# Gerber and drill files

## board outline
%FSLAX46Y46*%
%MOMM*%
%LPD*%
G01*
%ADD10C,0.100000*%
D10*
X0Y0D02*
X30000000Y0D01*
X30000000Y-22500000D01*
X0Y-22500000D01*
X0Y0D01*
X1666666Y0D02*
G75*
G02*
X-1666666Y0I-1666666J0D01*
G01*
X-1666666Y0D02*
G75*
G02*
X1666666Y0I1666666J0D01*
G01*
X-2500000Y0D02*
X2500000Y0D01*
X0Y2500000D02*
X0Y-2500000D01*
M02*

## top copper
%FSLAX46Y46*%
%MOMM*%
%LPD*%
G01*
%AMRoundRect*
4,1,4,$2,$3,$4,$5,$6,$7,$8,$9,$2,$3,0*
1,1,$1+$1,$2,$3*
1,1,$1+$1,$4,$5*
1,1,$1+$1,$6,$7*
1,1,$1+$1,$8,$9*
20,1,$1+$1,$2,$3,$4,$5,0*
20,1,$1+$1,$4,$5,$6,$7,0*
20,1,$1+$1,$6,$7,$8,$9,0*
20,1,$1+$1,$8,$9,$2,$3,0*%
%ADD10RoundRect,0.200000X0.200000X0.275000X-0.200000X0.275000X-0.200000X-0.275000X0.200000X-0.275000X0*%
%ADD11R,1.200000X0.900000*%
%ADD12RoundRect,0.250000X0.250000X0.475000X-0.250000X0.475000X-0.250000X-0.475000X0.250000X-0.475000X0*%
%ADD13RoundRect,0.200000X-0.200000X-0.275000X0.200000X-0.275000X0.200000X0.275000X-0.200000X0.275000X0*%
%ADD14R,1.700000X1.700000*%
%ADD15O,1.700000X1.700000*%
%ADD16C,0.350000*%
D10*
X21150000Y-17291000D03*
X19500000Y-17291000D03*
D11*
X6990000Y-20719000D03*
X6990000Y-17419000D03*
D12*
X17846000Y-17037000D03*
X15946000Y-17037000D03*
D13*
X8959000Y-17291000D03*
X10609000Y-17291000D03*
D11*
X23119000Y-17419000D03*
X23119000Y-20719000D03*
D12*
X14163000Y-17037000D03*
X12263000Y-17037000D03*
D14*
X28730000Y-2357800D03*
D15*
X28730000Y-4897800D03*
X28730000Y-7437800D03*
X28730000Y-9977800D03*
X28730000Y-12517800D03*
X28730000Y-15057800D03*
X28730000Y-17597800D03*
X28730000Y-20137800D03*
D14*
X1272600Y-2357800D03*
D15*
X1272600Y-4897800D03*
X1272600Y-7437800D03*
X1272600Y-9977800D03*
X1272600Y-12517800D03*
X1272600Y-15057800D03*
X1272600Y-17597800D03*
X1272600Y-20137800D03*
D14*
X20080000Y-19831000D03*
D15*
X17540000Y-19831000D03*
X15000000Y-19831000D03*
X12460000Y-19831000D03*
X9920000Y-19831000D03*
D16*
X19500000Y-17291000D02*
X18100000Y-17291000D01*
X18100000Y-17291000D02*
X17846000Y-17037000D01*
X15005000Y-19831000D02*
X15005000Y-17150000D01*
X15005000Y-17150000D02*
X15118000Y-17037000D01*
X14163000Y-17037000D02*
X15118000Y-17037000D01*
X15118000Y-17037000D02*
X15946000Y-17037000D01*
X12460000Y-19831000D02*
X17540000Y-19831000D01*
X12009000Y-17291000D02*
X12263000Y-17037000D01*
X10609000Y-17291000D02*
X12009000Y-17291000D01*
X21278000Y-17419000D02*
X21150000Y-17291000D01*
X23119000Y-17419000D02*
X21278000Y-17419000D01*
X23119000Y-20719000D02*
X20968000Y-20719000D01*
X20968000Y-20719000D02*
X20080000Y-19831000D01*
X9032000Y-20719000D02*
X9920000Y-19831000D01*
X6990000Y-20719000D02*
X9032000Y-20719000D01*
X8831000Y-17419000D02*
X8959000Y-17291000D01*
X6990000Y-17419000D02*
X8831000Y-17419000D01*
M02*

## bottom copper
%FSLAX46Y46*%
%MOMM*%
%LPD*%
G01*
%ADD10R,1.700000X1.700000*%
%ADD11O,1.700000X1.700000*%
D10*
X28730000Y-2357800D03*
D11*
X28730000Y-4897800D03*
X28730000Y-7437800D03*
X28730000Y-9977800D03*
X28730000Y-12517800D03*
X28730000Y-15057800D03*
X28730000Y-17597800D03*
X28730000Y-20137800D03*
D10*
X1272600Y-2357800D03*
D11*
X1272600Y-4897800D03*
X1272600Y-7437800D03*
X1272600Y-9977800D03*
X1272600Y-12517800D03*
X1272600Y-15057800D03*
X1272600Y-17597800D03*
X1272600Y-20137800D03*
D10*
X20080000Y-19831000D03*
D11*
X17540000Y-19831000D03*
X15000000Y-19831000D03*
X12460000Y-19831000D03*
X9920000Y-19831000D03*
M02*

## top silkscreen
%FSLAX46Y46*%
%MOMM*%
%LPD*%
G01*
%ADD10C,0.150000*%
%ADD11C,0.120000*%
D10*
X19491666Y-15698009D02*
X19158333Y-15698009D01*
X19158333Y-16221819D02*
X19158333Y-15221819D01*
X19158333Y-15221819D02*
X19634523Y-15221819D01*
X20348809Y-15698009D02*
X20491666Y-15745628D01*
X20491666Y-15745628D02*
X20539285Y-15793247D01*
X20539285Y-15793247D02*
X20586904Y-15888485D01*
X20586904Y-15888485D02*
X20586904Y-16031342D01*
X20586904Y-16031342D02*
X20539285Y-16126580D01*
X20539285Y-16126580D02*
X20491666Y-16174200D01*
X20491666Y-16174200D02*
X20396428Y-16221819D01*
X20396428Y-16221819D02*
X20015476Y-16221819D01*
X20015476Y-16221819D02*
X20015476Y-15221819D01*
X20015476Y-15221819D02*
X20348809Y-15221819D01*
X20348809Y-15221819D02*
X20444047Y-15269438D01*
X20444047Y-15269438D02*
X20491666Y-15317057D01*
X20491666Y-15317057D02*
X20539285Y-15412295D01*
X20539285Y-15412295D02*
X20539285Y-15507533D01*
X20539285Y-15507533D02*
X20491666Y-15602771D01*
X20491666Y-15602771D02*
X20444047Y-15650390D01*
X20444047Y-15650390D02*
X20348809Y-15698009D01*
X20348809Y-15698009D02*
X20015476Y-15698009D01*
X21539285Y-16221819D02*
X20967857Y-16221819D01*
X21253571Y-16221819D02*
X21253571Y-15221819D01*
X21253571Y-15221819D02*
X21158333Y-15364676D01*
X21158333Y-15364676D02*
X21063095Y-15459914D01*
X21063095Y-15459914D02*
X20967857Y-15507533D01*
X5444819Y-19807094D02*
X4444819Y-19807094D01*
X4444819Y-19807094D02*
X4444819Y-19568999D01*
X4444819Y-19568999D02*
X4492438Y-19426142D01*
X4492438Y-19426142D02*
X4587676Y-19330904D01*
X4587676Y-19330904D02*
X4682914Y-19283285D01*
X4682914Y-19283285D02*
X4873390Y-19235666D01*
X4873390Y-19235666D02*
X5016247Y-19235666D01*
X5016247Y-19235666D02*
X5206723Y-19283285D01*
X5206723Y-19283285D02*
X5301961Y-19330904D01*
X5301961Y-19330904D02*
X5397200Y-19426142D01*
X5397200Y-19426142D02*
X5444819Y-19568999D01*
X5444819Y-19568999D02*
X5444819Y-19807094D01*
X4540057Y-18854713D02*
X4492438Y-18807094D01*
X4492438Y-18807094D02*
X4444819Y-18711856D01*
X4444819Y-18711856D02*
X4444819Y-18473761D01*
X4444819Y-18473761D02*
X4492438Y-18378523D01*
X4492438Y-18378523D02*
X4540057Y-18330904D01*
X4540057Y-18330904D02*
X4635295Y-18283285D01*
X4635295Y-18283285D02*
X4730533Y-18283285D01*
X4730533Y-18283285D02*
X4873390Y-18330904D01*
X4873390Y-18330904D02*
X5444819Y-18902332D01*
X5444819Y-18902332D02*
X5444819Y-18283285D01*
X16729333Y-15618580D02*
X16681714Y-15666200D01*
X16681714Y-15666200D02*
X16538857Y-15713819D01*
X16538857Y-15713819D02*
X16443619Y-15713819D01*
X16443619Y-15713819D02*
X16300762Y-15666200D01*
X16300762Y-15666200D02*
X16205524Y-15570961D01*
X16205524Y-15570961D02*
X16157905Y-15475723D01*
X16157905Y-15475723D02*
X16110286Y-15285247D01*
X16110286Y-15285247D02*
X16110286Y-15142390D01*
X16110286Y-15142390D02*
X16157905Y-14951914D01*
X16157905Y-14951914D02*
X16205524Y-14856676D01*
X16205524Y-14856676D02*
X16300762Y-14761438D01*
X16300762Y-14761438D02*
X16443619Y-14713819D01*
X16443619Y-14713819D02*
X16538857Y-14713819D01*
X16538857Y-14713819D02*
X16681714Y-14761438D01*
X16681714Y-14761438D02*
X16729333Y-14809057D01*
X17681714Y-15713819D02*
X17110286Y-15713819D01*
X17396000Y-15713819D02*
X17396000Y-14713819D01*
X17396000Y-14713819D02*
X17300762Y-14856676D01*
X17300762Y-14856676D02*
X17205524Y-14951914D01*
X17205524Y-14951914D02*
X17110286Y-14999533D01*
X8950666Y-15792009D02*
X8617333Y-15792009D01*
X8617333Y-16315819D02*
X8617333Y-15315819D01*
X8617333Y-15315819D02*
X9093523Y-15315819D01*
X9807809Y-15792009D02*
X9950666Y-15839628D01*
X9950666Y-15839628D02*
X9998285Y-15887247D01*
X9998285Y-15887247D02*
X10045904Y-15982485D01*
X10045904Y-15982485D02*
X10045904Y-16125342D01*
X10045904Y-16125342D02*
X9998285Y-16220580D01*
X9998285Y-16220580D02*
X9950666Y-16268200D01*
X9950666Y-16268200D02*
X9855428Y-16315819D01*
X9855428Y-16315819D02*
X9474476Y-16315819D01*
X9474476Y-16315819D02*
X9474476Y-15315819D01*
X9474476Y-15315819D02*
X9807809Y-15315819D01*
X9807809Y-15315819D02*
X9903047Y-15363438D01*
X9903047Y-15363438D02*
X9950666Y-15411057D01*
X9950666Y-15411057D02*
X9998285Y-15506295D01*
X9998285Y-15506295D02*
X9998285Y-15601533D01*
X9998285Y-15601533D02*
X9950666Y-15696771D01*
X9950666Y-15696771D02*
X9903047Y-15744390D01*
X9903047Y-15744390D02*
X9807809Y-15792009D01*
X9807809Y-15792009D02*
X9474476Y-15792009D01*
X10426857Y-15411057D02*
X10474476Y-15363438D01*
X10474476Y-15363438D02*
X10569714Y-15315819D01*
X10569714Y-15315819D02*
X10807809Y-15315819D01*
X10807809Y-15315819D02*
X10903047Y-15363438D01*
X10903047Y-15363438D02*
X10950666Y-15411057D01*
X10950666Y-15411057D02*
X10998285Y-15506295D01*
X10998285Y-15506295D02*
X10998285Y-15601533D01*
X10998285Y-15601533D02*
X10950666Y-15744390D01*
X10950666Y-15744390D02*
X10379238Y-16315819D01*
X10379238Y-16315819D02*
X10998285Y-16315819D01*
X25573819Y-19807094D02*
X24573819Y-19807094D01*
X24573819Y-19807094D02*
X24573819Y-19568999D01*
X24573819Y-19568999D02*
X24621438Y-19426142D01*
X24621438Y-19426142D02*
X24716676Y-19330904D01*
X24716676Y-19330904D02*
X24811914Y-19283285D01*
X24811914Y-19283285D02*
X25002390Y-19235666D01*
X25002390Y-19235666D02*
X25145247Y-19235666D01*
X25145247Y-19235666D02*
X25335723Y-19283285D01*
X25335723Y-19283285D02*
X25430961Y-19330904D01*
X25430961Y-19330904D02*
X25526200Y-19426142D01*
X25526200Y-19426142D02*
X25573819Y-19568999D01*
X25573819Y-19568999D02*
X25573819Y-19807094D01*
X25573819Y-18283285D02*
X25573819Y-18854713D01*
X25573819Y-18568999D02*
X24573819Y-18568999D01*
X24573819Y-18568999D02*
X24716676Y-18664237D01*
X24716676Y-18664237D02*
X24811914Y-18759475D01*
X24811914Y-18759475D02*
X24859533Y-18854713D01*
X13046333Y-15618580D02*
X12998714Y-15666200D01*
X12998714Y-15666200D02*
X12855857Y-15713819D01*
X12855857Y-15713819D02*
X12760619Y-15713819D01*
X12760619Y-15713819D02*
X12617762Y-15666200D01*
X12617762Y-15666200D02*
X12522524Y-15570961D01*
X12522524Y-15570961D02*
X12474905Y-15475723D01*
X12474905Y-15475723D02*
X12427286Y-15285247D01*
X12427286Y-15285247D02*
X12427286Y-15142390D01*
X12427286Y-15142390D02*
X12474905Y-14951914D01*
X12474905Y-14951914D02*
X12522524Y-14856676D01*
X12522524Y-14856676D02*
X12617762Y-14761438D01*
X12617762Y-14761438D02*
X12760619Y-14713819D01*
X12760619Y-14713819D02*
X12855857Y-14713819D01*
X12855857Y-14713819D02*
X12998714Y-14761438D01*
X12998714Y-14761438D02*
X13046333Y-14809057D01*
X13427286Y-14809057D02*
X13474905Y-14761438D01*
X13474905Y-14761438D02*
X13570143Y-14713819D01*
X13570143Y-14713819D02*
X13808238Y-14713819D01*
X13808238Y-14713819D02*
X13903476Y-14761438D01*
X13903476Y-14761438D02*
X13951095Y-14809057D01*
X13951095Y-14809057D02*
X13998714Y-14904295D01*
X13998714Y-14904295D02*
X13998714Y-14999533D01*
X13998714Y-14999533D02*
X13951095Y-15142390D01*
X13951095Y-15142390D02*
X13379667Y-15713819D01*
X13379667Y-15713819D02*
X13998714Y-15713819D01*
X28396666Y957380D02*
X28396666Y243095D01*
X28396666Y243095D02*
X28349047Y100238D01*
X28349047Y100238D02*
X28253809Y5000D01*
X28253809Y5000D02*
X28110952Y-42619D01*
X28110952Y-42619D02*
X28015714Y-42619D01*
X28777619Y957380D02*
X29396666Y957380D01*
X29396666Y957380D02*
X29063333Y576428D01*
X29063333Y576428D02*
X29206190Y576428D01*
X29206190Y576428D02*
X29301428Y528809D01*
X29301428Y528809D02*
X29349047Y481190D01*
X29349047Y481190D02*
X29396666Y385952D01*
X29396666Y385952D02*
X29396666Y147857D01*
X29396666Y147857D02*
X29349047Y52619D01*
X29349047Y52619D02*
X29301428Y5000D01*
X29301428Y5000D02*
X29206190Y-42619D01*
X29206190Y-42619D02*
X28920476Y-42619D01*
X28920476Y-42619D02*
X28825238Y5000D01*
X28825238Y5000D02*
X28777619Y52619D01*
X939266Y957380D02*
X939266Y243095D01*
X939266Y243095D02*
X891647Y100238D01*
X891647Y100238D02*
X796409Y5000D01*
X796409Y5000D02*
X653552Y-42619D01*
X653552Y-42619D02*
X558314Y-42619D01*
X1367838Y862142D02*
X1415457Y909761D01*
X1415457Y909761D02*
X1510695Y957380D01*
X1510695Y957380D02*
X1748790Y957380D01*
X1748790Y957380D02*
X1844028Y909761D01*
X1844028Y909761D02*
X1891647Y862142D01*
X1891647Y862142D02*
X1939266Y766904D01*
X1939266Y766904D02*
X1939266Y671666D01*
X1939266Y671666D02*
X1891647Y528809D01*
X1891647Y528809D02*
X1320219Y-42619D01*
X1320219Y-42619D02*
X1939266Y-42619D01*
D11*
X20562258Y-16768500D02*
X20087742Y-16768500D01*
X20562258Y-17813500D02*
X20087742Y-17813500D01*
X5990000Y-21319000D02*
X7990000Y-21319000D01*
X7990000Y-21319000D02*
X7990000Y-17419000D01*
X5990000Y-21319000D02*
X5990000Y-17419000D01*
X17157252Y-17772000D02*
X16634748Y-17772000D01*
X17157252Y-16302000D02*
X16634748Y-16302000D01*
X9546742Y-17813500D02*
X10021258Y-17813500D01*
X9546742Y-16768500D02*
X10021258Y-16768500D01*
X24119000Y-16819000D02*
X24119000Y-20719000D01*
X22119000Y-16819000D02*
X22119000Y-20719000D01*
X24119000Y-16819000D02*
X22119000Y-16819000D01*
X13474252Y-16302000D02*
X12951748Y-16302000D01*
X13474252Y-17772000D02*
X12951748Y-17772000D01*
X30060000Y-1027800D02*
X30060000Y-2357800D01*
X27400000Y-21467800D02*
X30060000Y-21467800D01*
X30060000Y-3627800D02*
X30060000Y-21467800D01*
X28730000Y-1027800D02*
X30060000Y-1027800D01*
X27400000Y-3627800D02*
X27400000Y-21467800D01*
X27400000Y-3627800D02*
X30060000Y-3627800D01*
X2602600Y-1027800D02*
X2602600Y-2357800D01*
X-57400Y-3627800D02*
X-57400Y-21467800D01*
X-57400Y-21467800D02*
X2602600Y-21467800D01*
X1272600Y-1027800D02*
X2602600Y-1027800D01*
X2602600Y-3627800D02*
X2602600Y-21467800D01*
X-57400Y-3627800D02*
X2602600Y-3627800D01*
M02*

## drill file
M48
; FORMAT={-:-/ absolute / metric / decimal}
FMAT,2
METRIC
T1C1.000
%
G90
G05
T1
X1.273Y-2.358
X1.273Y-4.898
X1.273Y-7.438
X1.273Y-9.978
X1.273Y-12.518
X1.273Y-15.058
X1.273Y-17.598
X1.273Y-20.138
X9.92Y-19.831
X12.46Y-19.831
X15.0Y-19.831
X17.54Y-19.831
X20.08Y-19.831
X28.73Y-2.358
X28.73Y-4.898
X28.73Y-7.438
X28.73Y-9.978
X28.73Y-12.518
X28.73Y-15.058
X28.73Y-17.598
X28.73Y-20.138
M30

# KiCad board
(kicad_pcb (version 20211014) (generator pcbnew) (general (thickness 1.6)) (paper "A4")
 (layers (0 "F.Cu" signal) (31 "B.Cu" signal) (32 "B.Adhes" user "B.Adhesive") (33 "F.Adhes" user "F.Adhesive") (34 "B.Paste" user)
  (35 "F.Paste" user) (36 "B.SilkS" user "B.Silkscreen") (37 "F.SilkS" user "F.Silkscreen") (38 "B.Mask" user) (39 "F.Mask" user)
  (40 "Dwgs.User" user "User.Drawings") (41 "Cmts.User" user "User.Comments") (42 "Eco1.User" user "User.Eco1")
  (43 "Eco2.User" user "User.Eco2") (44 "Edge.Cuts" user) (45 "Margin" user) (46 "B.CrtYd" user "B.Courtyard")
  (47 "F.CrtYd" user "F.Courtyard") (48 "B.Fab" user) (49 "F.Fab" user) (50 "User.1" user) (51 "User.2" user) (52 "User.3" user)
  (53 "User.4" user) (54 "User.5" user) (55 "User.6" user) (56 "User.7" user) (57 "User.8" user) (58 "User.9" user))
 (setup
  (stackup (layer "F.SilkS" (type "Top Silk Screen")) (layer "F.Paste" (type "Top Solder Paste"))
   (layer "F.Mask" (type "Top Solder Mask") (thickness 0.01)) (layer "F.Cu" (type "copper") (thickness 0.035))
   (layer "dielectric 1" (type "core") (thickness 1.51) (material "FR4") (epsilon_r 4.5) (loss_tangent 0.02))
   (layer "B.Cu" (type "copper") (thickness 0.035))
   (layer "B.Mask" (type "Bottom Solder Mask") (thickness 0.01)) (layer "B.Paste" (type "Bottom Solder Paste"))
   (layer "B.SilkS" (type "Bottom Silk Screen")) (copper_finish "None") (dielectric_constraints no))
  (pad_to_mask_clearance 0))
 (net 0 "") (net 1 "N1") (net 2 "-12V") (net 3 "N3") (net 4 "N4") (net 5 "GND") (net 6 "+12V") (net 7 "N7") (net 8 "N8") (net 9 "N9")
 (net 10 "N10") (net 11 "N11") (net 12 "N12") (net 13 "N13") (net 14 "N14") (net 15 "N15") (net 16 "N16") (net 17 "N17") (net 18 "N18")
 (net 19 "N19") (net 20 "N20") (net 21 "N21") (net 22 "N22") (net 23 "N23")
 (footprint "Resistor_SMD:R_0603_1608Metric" (layer "F.Cu") (at 20.325 17.291 180)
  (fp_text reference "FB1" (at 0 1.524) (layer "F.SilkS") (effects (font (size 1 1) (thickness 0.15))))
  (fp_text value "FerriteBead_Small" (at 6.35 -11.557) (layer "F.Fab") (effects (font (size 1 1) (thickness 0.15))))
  (fp_line (start -0.237258 0.5225) (end 0.237258 0.5225) (layer "F.SilkS") (width 0.12))
  (fp_line (start -0.237258 -0.5225) (end 0.237258 -0.5225) (layer "F.SilkS") (width 0.12))
  (pad "1" smd roundrect (at -0.825 0 180) (size 0.8 0.95) (layers "F.Cu" "F.Paste" "F.Mask") (roundrect_rratio 0.25) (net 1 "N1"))
  (pad "2" smd roundrect (at 0.825 0 180) (size 0.8 0.95) (layers "F.Cu" "F.Paste" "F.Mask") (roundrect_rratio 0.25) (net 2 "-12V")))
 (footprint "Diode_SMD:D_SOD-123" (layer "F.Cu") (at 6.99 19.069 90)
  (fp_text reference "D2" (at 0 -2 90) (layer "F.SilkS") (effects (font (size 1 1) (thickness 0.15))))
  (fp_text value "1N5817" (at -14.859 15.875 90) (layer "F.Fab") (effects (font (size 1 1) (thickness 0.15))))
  (fp_line (start -2.25 -1) (end -2.25 1) (layer "F.SilkS") (width 0.12))
  (fp_line (start -2.25 1) (end 1.65 1) (layer "F.SilkS") (width 0.12))
  (fp_line (start -2.25 -1) (end 1.65 -1) (layer "F.SilkS") (width 0.12))
  (pad "1" smd rect (at -1.65 0 90) (size 0.9 1.2) (layers "F.Cu" "F.Paste" "F.Mask") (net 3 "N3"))
  (pad "2" smd rect (at 1.65 0 90) (size 0.9 1.2) (layers "F.Cu" "F.Paste" "F.Mask") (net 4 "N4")))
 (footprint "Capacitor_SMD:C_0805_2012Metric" (layer "F.Cu") (at 16.896 17.037 180)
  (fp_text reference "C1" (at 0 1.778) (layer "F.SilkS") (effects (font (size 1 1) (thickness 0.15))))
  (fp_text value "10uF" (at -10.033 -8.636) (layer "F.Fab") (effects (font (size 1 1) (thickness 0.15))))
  (fp_line (start -0.261252 -0.735) (end 0.261252 -0.735) (layer "F.SilkS") (width 0.12))
  (fp_line (start -0.261252 0.735) (end 0.261252 0.735) (layer "F.SilkS") (width 0.12))
  (pad "1" smd roundrect (at -0.95 0 180) (size 1 1.45) (layers "F.Cu" "F.Paste" "F.Mask") (roundrect_rratio 0.25) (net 2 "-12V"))
  (pad "2" smd roundrect (at 0.95 0 180) (size 1 1.45) (layers "F.Cu" "F.Paste" "F.Mask") (roundrect_rratio 0.25) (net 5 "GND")))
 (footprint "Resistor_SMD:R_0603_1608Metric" (layer "F.Cu") (at 9.784 17.291)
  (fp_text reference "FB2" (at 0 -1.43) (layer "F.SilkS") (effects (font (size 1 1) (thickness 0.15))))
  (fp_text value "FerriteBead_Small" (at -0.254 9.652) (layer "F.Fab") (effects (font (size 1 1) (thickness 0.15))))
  (fp_line (start -0.237258 0.5225) (end 0.237258 0.5225) (layer "F.SilkS") (width 0.12))
  (fp_line (start -0.237258 -0.5225) (end 0.237258 -0.5225) (layer "F.SilkS") (width 0.12))
  (pad "1" smd roundrect (at -0.825 0) (size 0.8 0.95) (layers "F.Cu" "F.Paste" "F.Mask") (roundrect_rratio 0.25) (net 4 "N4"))
  (pad "2" smd roundrect (at 0.825 0) (size 0.8 0.95) (layers "F.Cu" "F.Paste" "F.Mask") (roundrect_rratio 0.25) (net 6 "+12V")))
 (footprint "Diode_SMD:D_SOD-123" (layer "F.Cu") (at 23.119 19.069 -90)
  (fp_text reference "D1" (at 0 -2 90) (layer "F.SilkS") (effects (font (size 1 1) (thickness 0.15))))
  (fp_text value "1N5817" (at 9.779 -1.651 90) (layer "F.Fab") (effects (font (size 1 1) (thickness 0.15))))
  (fp_line (start -2.25 -1) (end 1.65 -1) (layer "F.SilkS") (width 0.12))
  (fp_line (start -2.25 1) (end 1.65 1) (layer "F.SilkS") (width 0.12))
  (fp_line (start -2.25 -1) (end -2.25 1) (layer "F.SilkS") (width 0.12))
  (pad "1" smd rect (at -1.65 0 270) (size 0.9 1.2) (layers "F.Cu" "F.Paste" "F.Mask") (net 1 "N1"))
  (pad "2" smd rect (at 1.65 0 270) (size 0.9 1.2) (layers "F.Cu" "F.Paste" "F.Mask") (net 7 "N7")))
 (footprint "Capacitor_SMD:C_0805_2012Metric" (layer "F.Cu") (at 13.213 17.037 180)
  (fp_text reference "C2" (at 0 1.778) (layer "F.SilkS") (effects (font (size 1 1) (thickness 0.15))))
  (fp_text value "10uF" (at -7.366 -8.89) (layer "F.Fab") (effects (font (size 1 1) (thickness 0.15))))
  (fp_line (start -0.261252 0.735) (end 0.261252 0.735) (layer "F.SilkS") (width 0.12))
  (fp_line (start -0.261252 -0.735) (end 0.261252 -0.735) (layer "F.SilkS") (width 0.12))
  (pad "1" smd roundrect (at -0.95 0 180) (size 1 1.45) (layers "F.Cu" "F.Paste" "F.Mask") (roundrect_rratio 0.25) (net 5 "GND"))
  (pad "2" smd roundrect (at 0.95 0 180) (size 1 1.45) (layers "F.Cu" "F.Paste" "F.Mask") (roundrect_rratio 0.25) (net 6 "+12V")))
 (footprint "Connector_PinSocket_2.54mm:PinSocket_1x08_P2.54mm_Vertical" (layer "F.Cu") (at 28.73 2.3578)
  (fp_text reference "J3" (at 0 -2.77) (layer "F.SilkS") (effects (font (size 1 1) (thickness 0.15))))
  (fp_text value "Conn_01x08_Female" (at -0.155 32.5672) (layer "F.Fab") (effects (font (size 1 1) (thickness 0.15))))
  (fp_line (start 1.33 -1.33) (end 1.33 0) (layer "F.SilkS") (width 0.12))
  (fp_line (start -1.33 19.11) (end 1.33 19.11) (layer "F.SilkS") (width 0.12))
  (fp_line (start 1.33 1.27) (end 1.33 19.11) (layer "F.SilkS") (width 0.12))
  (fp_line (start 0 -1.33) (end 1.33 -1.33) (layer "F.SilkS") (width 0.12))
  (fp_line (start -1.33 1.27) (end -1.33 19.11) (layer "F.SilkS") (width 0.12))
  (fp_line (start -1.33 1.27) (end 1.33 1.27) (layer "F.SilkS") (width 0.12))
  (pad "1" thru_hole rect (at 0 0) (size 1.7 1.7) (drill 1) (layers *.Cu *.Mask) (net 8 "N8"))
  (pad "2" thru_hole oval (at 0 2.54) (size 1.7 1.7) (drill 1) (layers *.Cu *.Mask) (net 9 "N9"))
  (pad "3" thru_hole oval (at 0 5.08) (size 1.7 1.7) (drill 1) (layers *.Cu *.Mask) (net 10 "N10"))
  (pad "4" thru_hole oval (at 0 7.62) (size 1.7 1.7) (drill 1) (layers *.Cu *.Mask) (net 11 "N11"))
  (pad "5" thru_hole oval (at 0 10.16) (size 1.7 1.7) (drill 1) (layers *.Cu *.Mask) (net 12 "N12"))
  (pad "6" thru_hole oval (at 0 12.7) (size 1.7 1.7) (drill 1) (layers *.Cu *.Mask) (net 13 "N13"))
  (pad "7" thru_hole oval (at 0 15.24) (size 1.7 1.7) (drill 1) (layers *.Cu *.Mask) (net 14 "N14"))
  (pad "8" thru_hole oval (at 0 17.78) (size 1.7 1.7) (drill 1) (layers *.Cu *.Mask) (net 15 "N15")))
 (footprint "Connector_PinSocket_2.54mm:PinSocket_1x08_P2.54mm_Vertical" (layer "F.Cu") (at 1.2726 2.3578)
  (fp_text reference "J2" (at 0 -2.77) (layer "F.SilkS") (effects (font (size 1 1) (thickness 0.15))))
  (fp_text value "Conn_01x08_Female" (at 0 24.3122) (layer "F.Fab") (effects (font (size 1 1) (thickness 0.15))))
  (fp_line (start 1.33 -1.33) (end 1.33 0) (layer "F.SilkS") (width 0.12))
  (fp_line (start -1.33 1.27) (end -1.33 19.11) (layer "F.SilkS") (width 0.12))
  (fp_line (start -1.33 19.11) (end 1.33 19.11) (layer "F.SilkS") (width 0.12))
  (fp_line (start 0 -1.33) (end 1.33 -1.33) (layer "F.SilkS") (width 0.12))
  (fp_line (start 1.33 1.27) (end 1.33 19.11) (layer "F.SilkS") (width 0.12))
  (fp_line (start -1.33 1.27) (end 1.33 1.27) (layer "F.SilkS") (width 0.12))
  (pad "1" thru_hole rect (at 0 0) (size 1.7 1.7) (drill 1) (layers *.Cu *.Mask) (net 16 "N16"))
  (pad "2" thru_hole oval (at 0 2.54) (size 1.7 1.7) (drill 1) (layers *.Cu *.Mask) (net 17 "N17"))
  (pad "3" thru_hole oval (at 0 5.08) (size 1.7 1.7) (drill 1) (layers *.Cu *.Mask) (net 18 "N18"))
  (pad "4" thru_hole oval (at 0 7.62) (size 1.7 1.7) (drill 1) (layers *.Cu *.Mask) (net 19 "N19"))
  (pad "5" thru_hole oval (at 0 10.16) (size 1.7 1.7) (drill 1) (layers *.Cu *.Mask) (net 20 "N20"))
  (pad "6" thru_hole oval (at 0 12.7) (size 1.7 1.7) (drill 1) (layers *.Cu *.Mask) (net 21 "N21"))
  (pad "7" thru_hole oval (at 0 15.24) (size 1.7 1.7) (drill 1) (layers *.Cu *.Mask) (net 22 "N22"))
  (pad "8" thru_hole oval (at 0 17.78) (size 1.7 1.7) (drill 1) (layers *.Cu *.Mask) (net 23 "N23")))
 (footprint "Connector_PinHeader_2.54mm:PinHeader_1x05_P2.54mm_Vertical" (layer "B.Cu") (at 20.08 19.831 90)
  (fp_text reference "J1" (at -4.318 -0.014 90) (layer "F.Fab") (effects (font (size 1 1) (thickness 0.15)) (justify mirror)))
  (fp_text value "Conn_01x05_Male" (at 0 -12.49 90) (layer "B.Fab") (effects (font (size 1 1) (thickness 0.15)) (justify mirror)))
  (pad "1" thru_hole rect (at 0 0 90) (size 1.7 1.7) (drill 1) (layers *.Cu *.Mask) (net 7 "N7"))
  (pad "2" thru_hole oval (at 0 -2.54 90) (size 1.7 1.7) (drill 1) (layers *.Cu *.Mask) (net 5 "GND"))
  (pad "3" thru_hole oval (at 0 -5.08 90) (size 1.7 1.7) (drill 1) (layers *.Cu *.Mask) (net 5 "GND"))
  (pad "4" thru_hole oval (at 0 -7.62 90) (size 1.7 1.7) (drill 1) (layers *.Cu *.Mask) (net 5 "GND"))
  (pad "5" thru_hole oval (at 0 -10.16 90) (size 1.7 1.7) (drill 1) (layers *.Cu *.Mask) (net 3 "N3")))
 (gr_rect (start 0 0) (end 30 22.5) (layer "Edge.Cuts") (width 0.1) (fill none))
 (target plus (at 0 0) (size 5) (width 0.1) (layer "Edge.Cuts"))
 (segment (start 19.5 17.291) (end 18.1 17.291) (width 0.35) (layer "F.Cu") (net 2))
 (segment (start 18.1 17.291) (end 17.846 17.037) (width 0.35) (layer "F.Cu") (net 2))
 (segment (start 15.005 19.831) (end 15.005 17.15) (width 0.35) (layer "F.Cu") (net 5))
 (segment (start 15.005 17.15) (end 15.118 17.037) (width 0.35) (layer "F.Cu") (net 5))
 (segment (start 14.163 17.037) (end 15.118 17.037) (width 0.35) (layer "F.Cu") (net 5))
 (segment (start 15.118 17.037) (end 15.946 17.037) (width 0.35) (layer "F.Cu") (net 5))
 (segment (start 12.46 19.831) (end 17.54 19.831) (width 0.35) (layer "F.Cu") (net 5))
 (segment (start 12.009 17.291) (end 12.263 17.037) (width 0.35) (layer "F.Cu") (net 6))
 (segment (start 10.609 17.291) (end 12.009 17.291) (width 0.35) (layer "F.Cu") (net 6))
 (segment (start 21.278 17.419) (end 21.15 17.291) (width 0.35) (layer "F.Cu") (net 1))
 (segment (start 23.119 17.419) (end 21.278 17.419) (width 0.35) (layer "F.Cu") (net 1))
 (segment (start 23.119 20.719) (end 20.968 20.719) (width 0.35) (layer "F.Cu") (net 7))
 (segment (start 20.968 20.719) (end 20.08 19.831) (width 0.35) (layer "F.Cu") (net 7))
 (segment (start 9.032 20.719) (end 9.92 19.831) (width 0.35) (layer "F.Cu") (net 3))
 (segment (start 6.99 20.719) (end 9.032 20.719) (width 0.35) (layer "F.Cu") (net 3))
 (segment (start 8.831 17.419) (end 8.959 17.291) (width 0.35) (layer "F.Cu") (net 4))
 (segment (start 6.99 17.419) (end 8.831 17.419) (width 0.35) (layer "F.Cu") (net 4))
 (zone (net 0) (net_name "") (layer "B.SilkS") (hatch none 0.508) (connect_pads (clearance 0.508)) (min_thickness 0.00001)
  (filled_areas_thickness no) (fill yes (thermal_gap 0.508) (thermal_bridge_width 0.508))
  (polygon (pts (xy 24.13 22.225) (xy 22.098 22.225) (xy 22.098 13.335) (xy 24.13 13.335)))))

